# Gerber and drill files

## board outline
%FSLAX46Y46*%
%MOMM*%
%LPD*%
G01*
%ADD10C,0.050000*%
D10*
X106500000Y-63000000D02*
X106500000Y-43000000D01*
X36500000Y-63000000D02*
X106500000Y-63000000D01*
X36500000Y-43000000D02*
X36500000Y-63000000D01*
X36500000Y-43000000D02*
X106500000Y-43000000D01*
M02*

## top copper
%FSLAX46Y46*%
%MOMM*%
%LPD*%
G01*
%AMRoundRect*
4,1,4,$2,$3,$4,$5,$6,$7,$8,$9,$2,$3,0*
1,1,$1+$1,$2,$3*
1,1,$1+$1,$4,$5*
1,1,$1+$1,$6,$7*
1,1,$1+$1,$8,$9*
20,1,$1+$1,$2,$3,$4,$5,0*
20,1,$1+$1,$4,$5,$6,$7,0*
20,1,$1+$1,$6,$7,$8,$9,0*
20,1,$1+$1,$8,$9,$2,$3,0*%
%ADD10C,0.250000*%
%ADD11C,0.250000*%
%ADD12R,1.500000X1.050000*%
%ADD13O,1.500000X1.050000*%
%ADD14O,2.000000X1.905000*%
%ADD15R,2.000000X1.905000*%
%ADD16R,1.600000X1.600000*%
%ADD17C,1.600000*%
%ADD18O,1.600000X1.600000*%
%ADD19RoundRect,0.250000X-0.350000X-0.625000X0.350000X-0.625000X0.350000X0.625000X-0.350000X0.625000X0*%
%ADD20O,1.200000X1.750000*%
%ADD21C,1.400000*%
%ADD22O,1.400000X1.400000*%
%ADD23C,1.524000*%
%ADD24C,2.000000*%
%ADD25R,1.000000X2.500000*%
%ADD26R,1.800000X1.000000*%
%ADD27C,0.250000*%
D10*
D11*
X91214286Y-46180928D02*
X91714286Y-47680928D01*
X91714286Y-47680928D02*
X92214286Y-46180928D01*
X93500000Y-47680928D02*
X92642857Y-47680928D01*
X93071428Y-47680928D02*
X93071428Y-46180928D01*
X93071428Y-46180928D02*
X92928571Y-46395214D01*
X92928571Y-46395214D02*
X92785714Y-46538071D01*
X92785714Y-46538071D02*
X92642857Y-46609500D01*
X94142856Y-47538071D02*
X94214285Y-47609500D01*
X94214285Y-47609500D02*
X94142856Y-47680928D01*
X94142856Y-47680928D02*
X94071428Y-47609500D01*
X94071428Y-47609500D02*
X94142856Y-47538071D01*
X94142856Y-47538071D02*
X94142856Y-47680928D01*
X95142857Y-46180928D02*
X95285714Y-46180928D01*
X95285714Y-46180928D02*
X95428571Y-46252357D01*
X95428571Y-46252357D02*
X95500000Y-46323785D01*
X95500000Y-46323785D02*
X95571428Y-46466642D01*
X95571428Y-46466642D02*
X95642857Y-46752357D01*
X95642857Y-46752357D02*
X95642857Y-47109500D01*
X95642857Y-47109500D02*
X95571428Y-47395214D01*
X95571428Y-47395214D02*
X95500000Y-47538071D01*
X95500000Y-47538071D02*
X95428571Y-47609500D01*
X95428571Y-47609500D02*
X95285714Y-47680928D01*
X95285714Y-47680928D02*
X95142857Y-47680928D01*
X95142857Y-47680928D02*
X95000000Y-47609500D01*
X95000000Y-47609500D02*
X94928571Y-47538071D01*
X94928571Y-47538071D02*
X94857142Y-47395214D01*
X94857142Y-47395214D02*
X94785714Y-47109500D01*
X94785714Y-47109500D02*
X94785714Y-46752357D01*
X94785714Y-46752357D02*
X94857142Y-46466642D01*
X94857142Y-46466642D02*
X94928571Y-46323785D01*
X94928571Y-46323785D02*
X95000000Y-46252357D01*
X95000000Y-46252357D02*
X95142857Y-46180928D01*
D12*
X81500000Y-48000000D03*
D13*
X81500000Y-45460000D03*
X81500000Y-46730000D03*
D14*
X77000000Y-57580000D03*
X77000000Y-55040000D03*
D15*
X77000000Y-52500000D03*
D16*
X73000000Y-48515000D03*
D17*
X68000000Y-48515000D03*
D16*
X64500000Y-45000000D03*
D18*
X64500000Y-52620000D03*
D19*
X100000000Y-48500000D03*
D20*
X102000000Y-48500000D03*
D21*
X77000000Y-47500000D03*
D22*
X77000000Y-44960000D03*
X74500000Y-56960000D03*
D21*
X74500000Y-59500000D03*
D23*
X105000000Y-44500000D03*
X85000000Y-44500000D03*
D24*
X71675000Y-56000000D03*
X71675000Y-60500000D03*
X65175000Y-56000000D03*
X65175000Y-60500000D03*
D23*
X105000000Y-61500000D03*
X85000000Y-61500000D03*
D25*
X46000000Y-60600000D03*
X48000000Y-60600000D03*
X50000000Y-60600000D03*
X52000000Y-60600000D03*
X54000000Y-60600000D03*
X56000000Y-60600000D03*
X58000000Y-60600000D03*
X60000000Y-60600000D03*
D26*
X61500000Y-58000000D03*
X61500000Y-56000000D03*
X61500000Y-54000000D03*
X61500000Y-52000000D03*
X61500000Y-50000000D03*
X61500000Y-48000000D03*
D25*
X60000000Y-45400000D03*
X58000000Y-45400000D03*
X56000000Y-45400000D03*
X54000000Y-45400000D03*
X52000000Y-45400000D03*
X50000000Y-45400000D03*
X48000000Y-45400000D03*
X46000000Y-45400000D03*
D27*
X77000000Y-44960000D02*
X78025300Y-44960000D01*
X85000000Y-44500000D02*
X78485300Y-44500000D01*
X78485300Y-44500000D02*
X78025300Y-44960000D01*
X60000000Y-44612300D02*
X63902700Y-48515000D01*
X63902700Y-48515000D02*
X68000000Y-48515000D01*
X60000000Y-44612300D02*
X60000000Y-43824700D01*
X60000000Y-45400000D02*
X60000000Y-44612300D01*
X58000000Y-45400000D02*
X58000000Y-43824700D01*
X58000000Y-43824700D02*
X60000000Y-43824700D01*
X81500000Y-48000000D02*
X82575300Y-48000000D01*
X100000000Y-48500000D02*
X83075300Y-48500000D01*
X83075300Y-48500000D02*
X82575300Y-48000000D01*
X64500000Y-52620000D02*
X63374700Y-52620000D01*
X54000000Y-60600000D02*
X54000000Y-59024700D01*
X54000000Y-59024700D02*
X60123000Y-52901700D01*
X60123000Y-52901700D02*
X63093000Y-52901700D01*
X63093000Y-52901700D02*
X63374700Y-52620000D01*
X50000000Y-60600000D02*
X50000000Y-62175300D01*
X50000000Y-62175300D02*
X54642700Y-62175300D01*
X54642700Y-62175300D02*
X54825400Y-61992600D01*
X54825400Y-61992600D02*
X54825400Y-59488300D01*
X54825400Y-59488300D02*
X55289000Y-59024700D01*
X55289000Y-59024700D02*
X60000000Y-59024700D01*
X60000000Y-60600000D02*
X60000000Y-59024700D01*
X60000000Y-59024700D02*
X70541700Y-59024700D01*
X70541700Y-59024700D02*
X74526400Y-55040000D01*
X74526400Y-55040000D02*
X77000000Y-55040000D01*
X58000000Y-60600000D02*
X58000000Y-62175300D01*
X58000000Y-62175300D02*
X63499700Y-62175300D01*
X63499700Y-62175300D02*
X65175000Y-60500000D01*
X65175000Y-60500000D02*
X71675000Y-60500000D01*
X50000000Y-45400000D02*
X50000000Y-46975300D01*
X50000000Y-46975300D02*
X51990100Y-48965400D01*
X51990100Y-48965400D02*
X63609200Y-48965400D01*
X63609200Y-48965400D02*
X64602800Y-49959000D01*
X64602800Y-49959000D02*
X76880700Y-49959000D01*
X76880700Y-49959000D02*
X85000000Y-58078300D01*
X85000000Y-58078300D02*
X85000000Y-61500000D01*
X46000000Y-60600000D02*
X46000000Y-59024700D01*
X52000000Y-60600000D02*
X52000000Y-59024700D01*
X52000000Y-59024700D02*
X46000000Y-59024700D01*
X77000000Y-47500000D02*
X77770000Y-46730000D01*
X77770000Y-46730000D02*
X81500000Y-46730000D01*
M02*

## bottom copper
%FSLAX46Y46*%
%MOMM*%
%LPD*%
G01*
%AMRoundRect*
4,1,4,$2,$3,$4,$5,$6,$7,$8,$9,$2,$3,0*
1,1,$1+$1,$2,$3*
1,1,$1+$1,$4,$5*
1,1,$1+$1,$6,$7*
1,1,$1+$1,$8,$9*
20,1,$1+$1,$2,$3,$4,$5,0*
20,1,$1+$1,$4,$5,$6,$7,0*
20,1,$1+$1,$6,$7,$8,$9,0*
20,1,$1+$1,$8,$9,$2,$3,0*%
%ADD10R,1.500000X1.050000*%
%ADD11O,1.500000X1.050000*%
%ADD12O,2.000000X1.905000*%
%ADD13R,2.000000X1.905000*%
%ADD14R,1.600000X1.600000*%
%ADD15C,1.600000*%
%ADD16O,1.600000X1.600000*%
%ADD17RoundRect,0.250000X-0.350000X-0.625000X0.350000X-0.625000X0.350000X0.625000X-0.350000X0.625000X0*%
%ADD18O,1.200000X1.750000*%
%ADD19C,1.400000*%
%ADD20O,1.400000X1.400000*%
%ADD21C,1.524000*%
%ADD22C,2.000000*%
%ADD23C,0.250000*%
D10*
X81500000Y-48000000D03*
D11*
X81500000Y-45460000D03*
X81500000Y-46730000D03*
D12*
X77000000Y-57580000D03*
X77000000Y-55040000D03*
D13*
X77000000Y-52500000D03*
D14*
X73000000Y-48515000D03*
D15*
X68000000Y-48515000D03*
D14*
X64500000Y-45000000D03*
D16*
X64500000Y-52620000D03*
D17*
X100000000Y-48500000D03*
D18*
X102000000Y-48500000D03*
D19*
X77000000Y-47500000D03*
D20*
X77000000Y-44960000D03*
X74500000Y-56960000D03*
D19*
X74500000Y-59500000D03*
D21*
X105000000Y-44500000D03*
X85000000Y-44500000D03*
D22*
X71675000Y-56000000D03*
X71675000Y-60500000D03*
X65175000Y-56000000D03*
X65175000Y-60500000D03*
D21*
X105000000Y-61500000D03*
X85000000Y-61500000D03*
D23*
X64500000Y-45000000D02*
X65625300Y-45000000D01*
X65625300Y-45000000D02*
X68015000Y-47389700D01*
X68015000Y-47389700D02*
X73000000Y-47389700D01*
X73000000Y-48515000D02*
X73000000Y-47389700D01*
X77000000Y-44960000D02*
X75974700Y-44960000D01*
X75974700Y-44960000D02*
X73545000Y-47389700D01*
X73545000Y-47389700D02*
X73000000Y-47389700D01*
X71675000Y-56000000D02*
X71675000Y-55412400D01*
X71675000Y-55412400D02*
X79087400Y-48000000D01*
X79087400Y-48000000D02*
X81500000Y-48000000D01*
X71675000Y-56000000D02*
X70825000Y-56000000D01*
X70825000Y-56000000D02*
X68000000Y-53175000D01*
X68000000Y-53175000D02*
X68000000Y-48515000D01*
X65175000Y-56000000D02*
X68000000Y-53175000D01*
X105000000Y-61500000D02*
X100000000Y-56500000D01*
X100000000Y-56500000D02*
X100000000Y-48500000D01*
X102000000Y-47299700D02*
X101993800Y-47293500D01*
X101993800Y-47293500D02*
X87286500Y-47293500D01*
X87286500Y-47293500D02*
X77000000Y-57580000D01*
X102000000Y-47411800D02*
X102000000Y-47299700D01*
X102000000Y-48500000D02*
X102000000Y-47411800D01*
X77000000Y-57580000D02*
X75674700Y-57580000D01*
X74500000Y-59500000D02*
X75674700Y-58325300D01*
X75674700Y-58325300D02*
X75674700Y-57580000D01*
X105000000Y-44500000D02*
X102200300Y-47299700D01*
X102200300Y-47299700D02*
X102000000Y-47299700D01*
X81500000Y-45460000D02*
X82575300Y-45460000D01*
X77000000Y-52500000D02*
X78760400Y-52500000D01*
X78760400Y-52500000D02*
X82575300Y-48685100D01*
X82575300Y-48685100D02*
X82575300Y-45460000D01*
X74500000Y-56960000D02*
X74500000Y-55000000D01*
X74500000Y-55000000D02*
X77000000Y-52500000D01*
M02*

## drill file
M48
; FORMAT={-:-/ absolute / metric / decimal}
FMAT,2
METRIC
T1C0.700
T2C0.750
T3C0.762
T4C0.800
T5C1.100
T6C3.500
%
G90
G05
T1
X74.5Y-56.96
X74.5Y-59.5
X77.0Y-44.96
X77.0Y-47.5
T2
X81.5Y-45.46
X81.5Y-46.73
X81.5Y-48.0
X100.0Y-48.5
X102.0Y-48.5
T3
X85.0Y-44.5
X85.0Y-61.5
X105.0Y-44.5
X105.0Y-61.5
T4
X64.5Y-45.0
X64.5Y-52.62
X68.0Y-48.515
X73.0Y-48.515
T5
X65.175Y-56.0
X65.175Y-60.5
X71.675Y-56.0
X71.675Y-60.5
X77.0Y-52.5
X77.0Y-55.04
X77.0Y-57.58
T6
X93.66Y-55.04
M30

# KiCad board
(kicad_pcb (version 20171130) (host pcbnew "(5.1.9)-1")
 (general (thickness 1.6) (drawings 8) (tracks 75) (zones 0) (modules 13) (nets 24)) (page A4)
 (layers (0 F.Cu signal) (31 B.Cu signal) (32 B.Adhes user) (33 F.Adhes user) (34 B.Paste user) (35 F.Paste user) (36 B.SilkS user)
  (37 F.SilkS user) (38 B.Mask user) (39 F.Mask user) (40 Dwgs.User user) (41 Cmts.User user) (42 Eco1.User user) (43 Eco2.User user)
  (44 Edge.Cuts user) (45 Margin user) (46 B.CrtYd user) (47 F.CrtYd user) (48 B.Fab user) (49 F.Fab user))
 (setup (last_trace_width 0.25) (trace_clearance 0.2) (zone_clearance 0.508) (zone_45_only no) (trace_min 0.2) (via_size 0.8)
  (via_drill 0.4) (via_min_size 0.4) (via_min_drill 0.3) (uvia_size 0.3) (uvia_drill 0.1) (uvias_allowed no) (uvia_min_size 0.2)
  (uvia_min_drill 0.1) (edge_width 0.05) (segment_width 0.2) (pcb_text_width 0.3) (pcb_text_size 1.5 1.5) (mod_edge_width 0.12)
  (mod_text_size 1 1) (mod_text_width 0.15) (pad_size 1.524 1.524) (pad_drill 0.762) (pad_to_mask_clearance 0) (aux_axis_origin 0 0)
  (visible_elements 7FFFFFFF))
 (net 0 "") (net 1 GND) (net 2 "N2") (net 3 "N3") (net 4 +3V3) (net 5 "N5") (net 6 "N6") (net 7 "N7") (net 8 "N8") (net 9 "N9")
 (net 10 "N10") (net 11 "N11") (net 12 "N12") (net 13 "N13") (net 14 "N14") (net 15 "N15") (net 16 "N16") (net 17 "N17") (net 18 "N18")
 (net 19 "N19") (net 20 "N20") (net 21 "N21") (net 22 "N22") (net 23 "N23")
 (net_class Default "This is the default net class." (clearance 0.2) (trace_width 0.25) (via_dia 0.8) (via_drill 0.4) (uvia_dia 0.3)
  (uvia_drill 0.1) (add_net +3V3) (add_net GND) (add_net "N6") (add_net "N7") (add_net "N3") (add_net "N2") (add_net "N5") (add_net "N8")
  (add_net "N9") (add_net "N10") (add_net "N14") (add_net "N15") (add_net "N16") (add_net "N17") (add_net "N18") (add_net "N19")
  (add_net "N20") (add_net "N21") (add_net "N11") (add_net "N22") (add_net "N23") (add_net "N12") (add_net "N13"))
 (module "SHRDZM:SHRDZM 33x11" (layer B.Cu) (at 54 50.5 180)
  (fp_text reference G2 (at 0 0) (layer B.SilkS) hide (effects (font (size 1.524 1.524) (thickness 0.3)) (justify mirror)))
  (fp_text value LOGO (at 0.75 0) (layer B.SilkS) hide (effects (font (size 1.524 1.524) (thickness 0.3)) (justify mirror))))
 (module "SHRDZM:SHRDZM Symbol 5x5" (layer F.Cu) (at 101 59.5)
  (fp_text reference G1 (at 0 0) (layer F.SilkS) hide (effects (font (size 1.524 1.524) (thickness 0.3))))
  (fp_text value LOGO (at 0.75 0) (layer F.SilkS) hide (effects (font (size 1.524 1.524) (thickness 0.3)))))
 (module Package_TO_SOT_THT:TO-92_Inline (layer F.Cu) (at 81.5 48 90)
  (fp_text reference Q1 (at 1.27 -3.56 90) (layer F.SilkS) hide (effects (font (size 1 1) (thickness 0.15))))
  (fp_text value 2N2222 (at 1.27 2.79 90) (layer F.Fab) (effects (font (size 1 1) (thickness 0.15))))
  (pad 1 thru_hole rect (at 0 0 90) (size 1.05 1.5) (drill 0.75) (layers *.Cu *.Mask) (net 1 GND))
  (pad 3 thru_hole oval (at 2.54 0 90) (size 1.05 1.5) (drill 0.75) (layers *.Cu *.Mask) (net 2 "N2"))
  (pad 2 thru_hole oval (at 1.27 0 90) (size 1.05 1.5) (drill 0.75) (layers *.Cu *.Mask) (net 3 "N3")))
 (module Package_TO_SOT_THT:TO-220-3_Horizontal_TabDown (layer F.Cu) (at 77 52.5 270)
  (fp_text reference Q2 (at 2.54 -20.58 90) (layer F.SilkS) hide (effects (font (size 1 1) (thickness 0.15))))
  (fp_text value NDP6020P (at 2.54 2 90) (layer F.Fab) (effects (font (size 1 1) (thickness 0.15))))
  (pad 3 thru_hole oval (at 5.08 0 270) (size 1.905 2) (drill 1.1) (layers *.Cu *.Mask) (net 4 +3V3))
  (pad 2 thru_hole oval (at 2.54 0 270) (size 1.905 2) (drill 1.1) (layers *.Cu *.Mask) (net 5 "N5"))
  (pad 1 thru_hole rect (at 0 0 270) (size 1.905 2) (drill 1.1) (layers *.Cu *.Mask) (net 2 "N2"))
  (pad "" np_thru_hole oval (at 2.54 -16.66 270) (size 3.5 3.5) (drill 3.5) (layers *.Cu *.Mask)))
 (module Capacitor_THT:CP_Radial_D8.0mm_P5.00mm (layer F.Cu) (at 73 48.515 180)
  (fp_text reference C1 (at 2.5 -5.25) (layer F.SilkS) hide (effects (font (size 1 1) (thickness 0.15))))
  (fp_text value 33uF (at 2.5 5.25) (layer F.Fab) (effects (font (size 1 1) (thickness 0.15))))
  (pad 1 thru_hole rect (at 0 0 180) (size 1.6 1.6) (drill 0.8) (layers *.Cu *.Mask) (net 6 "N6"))
  (pad 2 thru_hole circle (at 5 0 180) (size 1.6 1.6) (drill 0.8) (layers *.Cu *.Mask) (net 1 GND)))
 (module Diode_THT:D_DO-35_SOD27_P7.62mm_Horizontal (layer F.Cu) (at 64.5 45 270)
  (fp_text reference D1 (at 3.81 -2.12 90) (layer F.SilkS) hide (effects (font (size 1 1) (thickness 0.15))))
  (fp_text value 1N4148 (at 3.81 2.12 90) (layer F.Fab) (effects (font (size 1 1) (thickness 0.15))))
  (pad 1 thru_hole rect (at 0 0 270) (size 1.6 1.6) (drill 0.8) (layers *.Cu *.Mask) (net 6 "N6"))
  (pad 2 thru_hole oval (at 7.62 0 270) (size 1.6 1.6) (drill 0.8) (layers *.Cu *.Mask) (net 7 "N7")))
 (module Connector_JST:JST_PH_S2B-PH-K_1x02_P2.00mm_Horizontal (layer F.Cu) (at 100 48.5)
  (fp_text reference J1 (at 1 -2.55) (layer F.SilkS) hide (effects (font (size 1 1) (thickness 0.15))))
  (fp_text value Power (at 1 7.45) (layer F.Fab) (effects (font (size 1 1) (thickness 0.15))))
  (pad 1 thru_hole roundrect (at 0 0) (size 1.2 1.75) (drill 0.75) (layers *.Cu *.Mask) (roundrect_rratio 0.208333) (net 1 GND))
  (pad 2 thru_hole oval (at 2 0) (size 1.2 1.75) (drill 0.75) (layers *.Cu *.Mask) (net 4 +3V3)))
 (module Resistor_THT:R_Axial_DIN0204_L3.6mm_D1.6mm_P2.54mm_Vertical (layer F.Cu) (at 77 47.5 90)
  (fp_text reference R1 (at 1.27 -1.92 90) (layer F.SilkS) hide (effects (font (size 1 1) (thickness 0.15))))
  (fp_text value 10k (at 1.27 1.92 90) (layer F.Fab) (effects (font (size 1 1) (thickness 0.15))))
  (pad 1 thru_hole circle (at 0 0 90) (size 1.4 1.4) (drill 0.7) (layers *.Cu *.Mask) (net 3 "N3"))
  (pad 2 thru_hole oval (at 2.54 0 90) (size 1.4 1.4) (drill 0.7) (layers *.Cu *.Mask) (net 6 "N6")))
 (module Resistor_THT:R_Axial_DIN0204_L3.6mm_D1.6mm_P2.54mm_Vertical (layer F.Cu) (at 74.5 59.5 90)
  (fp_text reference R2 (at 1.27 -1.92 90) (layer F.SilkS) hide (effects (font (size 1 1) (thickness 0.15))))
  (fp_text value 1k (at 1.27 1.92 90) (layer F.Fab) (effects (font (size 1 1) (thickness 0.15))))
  (pad 2 thru_hole oval (at 2.54 0 90) (size 1.4 1.4) (drill 0.7) (layers *.Cu *.Mask) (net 2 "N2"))
  (pad 1 thru_hole circle (at 0 0 90) (size 1.4 1.4) (drill 0.7) (layers *.Cu *.Mask) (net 4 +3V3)))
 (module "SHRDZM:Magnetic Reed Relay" (layer F.Cu) (at 95 44.5 180)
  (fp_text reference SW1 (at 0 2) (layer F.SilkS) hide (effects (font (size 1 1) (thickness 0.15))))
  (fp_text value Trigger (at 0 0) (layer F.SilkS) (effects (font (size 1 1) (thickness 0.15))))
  (pad 1 thru_hole circle (at -10 0 180) (size 1.524 1.524) (drill 0.762) (layers *.Cu *.Mask) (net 4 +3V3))
  (pad 2 thru_hole circle (at 10 0 180) (size 1.524 1.524) (drill 0.762) (layers *.Cu *.Mask) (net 6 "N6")))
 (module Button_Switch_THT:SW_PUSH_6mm (layer F.Cu) (at 71.675 60.5 180)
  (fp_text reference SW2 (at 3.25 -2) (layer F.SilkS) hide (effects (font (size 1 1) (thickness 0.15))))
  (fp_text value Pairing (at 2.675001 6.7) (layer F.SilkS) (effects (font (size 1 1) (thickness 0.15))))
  (pad 2 thru_hole circle (at 0 4.5 270) (size 2 2) (drill 1.1) (layers *.Cu *.Mask) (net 1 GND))
  (pad 1 thru_hole circle (at 0 0 270) (size 2 2) (drill 1.1) (layers *.Cu *.Mask) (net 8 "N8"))
  (pad 2 thru_hole circle (at 6.5 4.5 270) (size 2 2) (drill 1.1) (layers *.Cu *.Mask) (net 1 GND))
  (pad 1 thru_hole circle (at 6.5 0 270) (size 2 2) (drill 1.1) (layers *.Cu *.Mask) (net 8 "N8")))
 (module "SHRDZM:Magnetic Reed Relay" (layer B.Cu) (at 95 61.5)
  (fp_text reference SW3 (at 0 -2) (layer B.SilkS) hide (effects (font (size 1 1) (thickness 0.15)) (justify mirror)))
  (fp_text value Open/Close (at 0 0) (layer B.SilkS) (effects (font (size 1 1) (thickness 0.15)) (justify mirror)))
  (pad 2 thru_hole circle (at 10 0) (size 1.524 1.524) (drill 0.762) (layers *.Cu *.Mask) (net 1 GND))
  (pad 1 thru_hole circle (at -10 0) (size 1.524 1.524) (drill 0.762) (layers *.Cu *.Mask) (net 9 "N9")))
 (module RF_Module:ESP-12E (layer F.Cu) (at 49.5 53 90)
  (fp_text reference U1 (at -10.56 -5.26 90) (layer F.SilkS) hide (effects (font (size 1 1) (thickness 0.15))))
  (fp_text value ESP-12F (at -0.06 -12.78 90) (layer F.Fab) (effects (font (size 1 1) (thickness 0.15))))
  (pad 1 smd rect (at -7.6 -3.5 90) (size 2.5 1) (layers F.Cu F.Paste F.Mask) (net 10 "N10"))
  (pad 2 smd rect (at -7.6 -1.5 90) (size 2.5 1) (layers F.Cu F.Paste F.Mask) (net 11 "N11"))
  (pad 3 smd rect (at -7.6 0.5 90) (size 2.5 1) (layers F.Cu F.Paste F.Mask) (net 5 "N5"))
  (pad 4 smd rect (at -7.6 2.5 90) (size 2.5 1) (layers F.Cu F.Paste F.Mask) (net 10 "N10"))
  (pad 5 smd rect (at -7.6 4.5 90) (size 2.5 1) (layers F.Cu F.Paste F.Mask) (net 7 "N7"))
  (pad 6 smd rect (at -7.6 6.5 90) (size 2.5 1) (layers F.Cu F.Paste F.Mask) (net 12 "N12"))
  (pad 7 smd rect (at -7.6 8.5 90) (size 2.5 1) (layers F.Cu F.Paste F.Mask) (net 8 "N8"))
  (pad 8 smd rect (at -7.6 10.5 90) (size 2.5 1) (layers F.Cu F.Paste F.Mask) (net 5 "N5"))
  (pad 9 smd rect (at -5 12 90) (size 1 1.8) (layers F.Cu F.Paste F.Mask) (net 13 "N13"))
  (pad 10 smd rect (at -3 12 90) (size 1 1.8) (layers F.Cu F.Paste F.Mask) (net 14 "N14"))
  (pad 11 smd rect (at -1 12 90) (size 1 1.8) (layers F.Cu F.Paste F.Mask) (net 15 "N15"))
  (pad 12 smd rect (at 1 12 90) (size 1 1.8) (layers F.Cu F.Paste F.Mask) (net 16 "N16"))
  (pad 13 smd rect (at 3 12 90) (size 1 1.8) (layers F.Cu F.Paste F.Mask) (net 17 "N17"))
  (pad 14 smd rect (at 5 12 90) (size 1 1.8) (layers F.Cu F.Paste F.Mask) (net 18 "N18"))
  (pad 15 smd rect (at 7.6 10.5 90) (size 2.5 1) (layers F.Cu F.Paste F.Mask) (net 1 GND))
  (pad 16 smd rect (at 7.6 8.5 90) (size 2.5 1) (layers F.Cu F.Paste F.Mask) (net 1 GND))
  (pad 17 smd rect (at 7.6 6.5 90) (size 2.5 1) (layers F.Cu F.Paste F.Mask) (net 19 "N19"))
  (pad 18 smd rect (at 7.6 4.5 90) (size 2.5 1) (layers F.Cu F.Paste F.Mask) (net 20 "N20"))
  (pad 19 smd rect (at 7.6 2.5 90) (size 2.5 1) (layers F.Cu F.Paste F.Mask) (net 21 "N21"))
  (pad 20 smd rect (at 7.6 0.5 90) (size 2.5 1) (layers F.Cu F.Paste F.Mask) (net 9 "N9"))
  (pad 21 smd rect (at 7.6 -1.5 90) (size 2.5 1) (layers F.Cu F.Paste F.Mask) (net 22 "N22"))
  (pad 22 smd rect (at 7.6 -3.5 90) (size 2.5 1) (layers F.Cu F.Paste F.Mask) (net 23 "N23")))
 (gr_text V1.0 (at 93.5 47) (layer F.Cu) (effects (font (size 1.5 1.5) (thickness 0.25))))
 (gr_line (start 106.5 63) (end 106.5 43) (layer Edge.Cuts) (width 0.05))
 (gr_line (start 36.5 63) (end 106.5 63) (layer Edge.Cuts) (width 0.05))
 (gr_line (start 36.5 43) (end 36.5 63) (layer Edge.Cuts) (width 0.05))
 (gr_line (start 36.5 43) (end 106.5 43) (layer Edge.Cuts) (width 0.05))
 (segment (start 64.5 45) (end 65.6253 45) (width 0.25) (layer B.Cu) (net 6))
 (segment (start 65.6253 45) (end 68.015 47.3897) (width 0.25) (layer B.Cu) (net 6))
 (segment (start 68.015 47.3897) (end 73 47.3897) (width 0.25) (layer B.Cu) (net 6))
 (segment (start 73 48.515) (end 73 47.3897) (width 0.25) (layer B.Cu) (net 6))
 (segment (start 77 44.96) (end 75.9747 44.96) (width 0.25) (layer B.Cu) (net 6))
 (segment (start 75.9747 44.96) (end 73.545 47.3897) (width 0.25) (layer B.Cu) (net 6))
 (segment (start 73.545 47.3897) (end 73 47.3897) (width 0.25) (layer B.Cu) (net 6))
 (segment (start 77 44.96) (end 78.0253 44.96) (width 0.25) (layer F.Cu) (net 6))
 (segment (start 85 44.5) (end 78.4853 44.5) (width 0.25) (layer F.Cu) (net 6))
 (segment (start 78.4853 44.5) (end 78.0253 44.96) (width 0.25) (layer F.Cu) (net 6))
 (segment (start 60 44.6123) (end 63.9027 48.515) (width 0.25) (layer F.Cu) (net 1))
 (segment (start 63.9027 48.515) (end 68 48.515) (width 0.25) (layer F.Cu) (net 1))
 (segment (start 60 44.6123) (end 60 43.8247) (width 0.25) (layer F.Cu) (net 1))
 (segment (start 60 45.4) (end 60 44.6123) (width 0.25) (layer F.Cu) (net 1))
 (segment (start 58 45.4) (end 58 43.8247) (width 0.25) (layer F.Cu) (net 1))
 (segment (start 58 43.8247) (end 60 43.8247) (width 0.25) (layer F.Cu) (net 1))
 (segment (start 71.675 56) (end 71.675 55.4124) (width 0.25) (layer B.Cu) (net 1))
 (segment (start 71.675 55.4124) (end 79.0874 48) (width 0.25) (layer B.Cu) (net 1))
 (segment (start 79.0874 48) (end 81.5 48) (width 0.25) (layer B.Cu) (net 1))
 (segment (start 71.675 56) (end 70.825 56) (width 0.25) (layer B.Cu) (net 1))
 (segment (start 70.825 56) (end 68 53.175) (width 0.25) (layer B.Cu) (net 1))
 (segment (start 81.5 48) (end 82.5753 48) (width 0.25) (layer F.Cu) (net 1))
 (segment (start 100 48.5) (end 83.0753 48.5) (width 0.25) (layer F.Cu) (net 1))
 (segment (start 83.0753 48.5) (end 82.5753 48) (width 0.25) (layer F.Cu) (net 1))
 (segment (start 68 53.175) (end 68 48.515) (width 0.25) (layer B.Cu) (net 1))
 (segment (start 65.175 56) (end 68 53.175) (width 0.25) (layer B.Cu) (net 1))
 (segment (start 105 61.5) (end 100 56.5) (width 0.25) (layer B.Cu) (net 1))
 (segment (start 100 56.5) (end 100 48.5) (width 0.25) (layer B.Cu) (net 1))
 (segment (start 64.5 52.62) (end 63.3747 52.62) (width 0.25) (layer F.Cu) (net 7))
 (segment (start 54 60.6) (end 54 59.0247) (width 0.25) (layer F.Cu) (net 7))
 (segment (start 54 59.0247) (end 60.123 52.9017) (width 0.25) (layer F.Cu) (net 7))
 (segment (start 60.123 52.9017) (end 63.093 52.9017) (width 0.25) (layer F.Cu) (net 7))
 (segment (start 63.093 52.9017) (end 63.3747 52.62) (width 0.25) (layer F.Cu) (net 7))
 (segment (start 102 47.2997) (end 101.9938 47.2935) (width 0.25) (layer B.Cu) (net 4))
 (segment (start 101.9938 47.2935) (end 87.2865 47.2935) (width 0.25) (layer B.Cu) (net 4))
 (segment (start 87.2865 47.2935) (end 77 57.58) (width 0.25) (layer B.Cu) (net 4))
 (segment (start 102 47.4118) (end 102 47.2997) (width 0.25) (layer B.Cu) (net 4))
 (segment (start 102 48.5) (end 102 47.4118) (width 0.25) (layer B.Cu) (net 4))
 (segment (start 77 57.58) (end 75.6747 57.58) (width 0.25) (layer B.Cu) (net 4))
 (segment (start 74.5 59.5) (end 75.6747 58.3253) (width 0.25) (layer B.Cu) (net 4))
 (segment (start 75.6747 58.3253) (end 75.6747 57.58) (width 0.25) (layer B.Cu) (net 4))
 (segment (start 105 44.5) (end 102.2003 47.2997) (width 0.25) (layer B.Cu) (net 4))
 (segment (start 102.2003 47.2997) (end 102 47.2997) (width 0.25) (layer B.Cu) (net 4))
 (segment (start 50 60.6) (end 50 62.1753) (width 0.25) (layer F.Cu) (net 5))
 (segment (start 50 62.1753) (end 54.6427 62.1753) (width 0.25) (layer F.Cu) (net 5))
 (segment (start 54.6427 62.1753) (end 54.8254 61.9926) (width 0.25) (layer F.Cu) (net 5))
 (segment (start 54.8254 61.9926) (end 54.8254 59.4883) (width 0.25) (layer F.Cu) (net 5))
 (segment (start 54.8254 59.4883) (end 55.289 59.0247) (width 0.25) (layer F.Cu) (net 5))
 (segment (start 55.289 59.0247) (end 60 59.0247) (width 0.25) (layer F.Cu) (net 5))
 (segment (start 60 60.6) (end 60 59.0247) (width 0.25) (layer F.Cu) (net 5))
 (segment (start 60 59.0247) (end 70.5417 59.0247) (width 0.25) (layer F.Cu) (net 5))
 (segment (start 70.5417 59.0247) (end 74.5264 55.04) (width 0.25) (layer F.Cu) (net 5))
 (segment (start 74.5264 55.04) (end 77 55.04) (width 0.25) (layer F.Cu) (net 5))
 (segment (start 58 60.6) (end 58 62.1753) (width 0.25) (layer F.Cu) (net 8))
 (segment (start 58 62.1753) (end 63.4997 62.1753) (width 0.25) (layer F.Cu) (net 8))
 (segment (start 63.4997 62.1753) (end 65.175 60.5) (width 0.25) (layer F.Cu) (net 8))
 (segment (start 65.175 60.5) (end 71.675 60.5) (width 0.25) (layer F.Cu) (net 8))
 (segment (start 50 45.4) (end 50 46.9753) (width 0.25) (layer F.Cu) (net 9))
 (segment (start 50 46.9753) (end 51.9901 48.9654) (width 0.25) (layer F.Cu) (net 9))
 (segment (start 51.9901 48.9654) (end 63.6092 48.9654) (width 0.25) (layer F.Cu) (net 9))
 (segment (start 63.6092 48.9654) (end 64.6028 49.959) (width 0.25) (layer F.Cu) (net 9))
 (segment (start 64.6028 49.959) (end 76.8807 49.959) (width 0.25) (layer F.Cu) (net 9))
 (segment (start 76.8807 49.959) (end 85 58.0783) (width 0.25) (layer F.Cu) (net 9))
 (segment (start 85 58.0783) (end 85 61.5) (width 0.25) (layer F.Cu) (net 9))
 (segment (start 46 60.6) (end 46 59.0247) (width 0.25) (layer F.Cu) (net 10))
 (segment (start 52 60.6) (end 52 59.0247) (width 0.25) (layer F.Cu) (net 10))
 (segment (start 52 59.0247) (end 46 59.0247) (width 0.25) (layer F.Cu) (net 10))
 (segment (start 77 47.5) (end 77.77 46.73) (width 0.25) (layer F.Cu) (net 3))
 (segment (start 77.77 46.73) (end 81.5 46.73) (width 0.25) (layer F.Cu) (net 3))
 (segment (start 81.5 45.46) (end 82.5753 45.46) (width 0.25) (layer B.Cu) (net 2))
 (segment (start 77 52.5) (end 78.7604 52.5) (width 0.25) (layer B.Cu) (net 2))
 (segment (start 78.7604 52.5) (end 82.5753 48.6851) (width 0.25) (layer B.Cu) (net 2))
 (segment (start 82.5753 48.6851) (end 82.5753 45.46) (width 0.25) (layer B.Cu) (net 2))
 (segment (start 74.5 56.96) (end 74.5 55) (width 0.25) (layer B.Cu) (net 2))
 (segment (start 74.5 55) (end 77 52.5) (width 0.25) (layer B.Cu) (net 2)))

